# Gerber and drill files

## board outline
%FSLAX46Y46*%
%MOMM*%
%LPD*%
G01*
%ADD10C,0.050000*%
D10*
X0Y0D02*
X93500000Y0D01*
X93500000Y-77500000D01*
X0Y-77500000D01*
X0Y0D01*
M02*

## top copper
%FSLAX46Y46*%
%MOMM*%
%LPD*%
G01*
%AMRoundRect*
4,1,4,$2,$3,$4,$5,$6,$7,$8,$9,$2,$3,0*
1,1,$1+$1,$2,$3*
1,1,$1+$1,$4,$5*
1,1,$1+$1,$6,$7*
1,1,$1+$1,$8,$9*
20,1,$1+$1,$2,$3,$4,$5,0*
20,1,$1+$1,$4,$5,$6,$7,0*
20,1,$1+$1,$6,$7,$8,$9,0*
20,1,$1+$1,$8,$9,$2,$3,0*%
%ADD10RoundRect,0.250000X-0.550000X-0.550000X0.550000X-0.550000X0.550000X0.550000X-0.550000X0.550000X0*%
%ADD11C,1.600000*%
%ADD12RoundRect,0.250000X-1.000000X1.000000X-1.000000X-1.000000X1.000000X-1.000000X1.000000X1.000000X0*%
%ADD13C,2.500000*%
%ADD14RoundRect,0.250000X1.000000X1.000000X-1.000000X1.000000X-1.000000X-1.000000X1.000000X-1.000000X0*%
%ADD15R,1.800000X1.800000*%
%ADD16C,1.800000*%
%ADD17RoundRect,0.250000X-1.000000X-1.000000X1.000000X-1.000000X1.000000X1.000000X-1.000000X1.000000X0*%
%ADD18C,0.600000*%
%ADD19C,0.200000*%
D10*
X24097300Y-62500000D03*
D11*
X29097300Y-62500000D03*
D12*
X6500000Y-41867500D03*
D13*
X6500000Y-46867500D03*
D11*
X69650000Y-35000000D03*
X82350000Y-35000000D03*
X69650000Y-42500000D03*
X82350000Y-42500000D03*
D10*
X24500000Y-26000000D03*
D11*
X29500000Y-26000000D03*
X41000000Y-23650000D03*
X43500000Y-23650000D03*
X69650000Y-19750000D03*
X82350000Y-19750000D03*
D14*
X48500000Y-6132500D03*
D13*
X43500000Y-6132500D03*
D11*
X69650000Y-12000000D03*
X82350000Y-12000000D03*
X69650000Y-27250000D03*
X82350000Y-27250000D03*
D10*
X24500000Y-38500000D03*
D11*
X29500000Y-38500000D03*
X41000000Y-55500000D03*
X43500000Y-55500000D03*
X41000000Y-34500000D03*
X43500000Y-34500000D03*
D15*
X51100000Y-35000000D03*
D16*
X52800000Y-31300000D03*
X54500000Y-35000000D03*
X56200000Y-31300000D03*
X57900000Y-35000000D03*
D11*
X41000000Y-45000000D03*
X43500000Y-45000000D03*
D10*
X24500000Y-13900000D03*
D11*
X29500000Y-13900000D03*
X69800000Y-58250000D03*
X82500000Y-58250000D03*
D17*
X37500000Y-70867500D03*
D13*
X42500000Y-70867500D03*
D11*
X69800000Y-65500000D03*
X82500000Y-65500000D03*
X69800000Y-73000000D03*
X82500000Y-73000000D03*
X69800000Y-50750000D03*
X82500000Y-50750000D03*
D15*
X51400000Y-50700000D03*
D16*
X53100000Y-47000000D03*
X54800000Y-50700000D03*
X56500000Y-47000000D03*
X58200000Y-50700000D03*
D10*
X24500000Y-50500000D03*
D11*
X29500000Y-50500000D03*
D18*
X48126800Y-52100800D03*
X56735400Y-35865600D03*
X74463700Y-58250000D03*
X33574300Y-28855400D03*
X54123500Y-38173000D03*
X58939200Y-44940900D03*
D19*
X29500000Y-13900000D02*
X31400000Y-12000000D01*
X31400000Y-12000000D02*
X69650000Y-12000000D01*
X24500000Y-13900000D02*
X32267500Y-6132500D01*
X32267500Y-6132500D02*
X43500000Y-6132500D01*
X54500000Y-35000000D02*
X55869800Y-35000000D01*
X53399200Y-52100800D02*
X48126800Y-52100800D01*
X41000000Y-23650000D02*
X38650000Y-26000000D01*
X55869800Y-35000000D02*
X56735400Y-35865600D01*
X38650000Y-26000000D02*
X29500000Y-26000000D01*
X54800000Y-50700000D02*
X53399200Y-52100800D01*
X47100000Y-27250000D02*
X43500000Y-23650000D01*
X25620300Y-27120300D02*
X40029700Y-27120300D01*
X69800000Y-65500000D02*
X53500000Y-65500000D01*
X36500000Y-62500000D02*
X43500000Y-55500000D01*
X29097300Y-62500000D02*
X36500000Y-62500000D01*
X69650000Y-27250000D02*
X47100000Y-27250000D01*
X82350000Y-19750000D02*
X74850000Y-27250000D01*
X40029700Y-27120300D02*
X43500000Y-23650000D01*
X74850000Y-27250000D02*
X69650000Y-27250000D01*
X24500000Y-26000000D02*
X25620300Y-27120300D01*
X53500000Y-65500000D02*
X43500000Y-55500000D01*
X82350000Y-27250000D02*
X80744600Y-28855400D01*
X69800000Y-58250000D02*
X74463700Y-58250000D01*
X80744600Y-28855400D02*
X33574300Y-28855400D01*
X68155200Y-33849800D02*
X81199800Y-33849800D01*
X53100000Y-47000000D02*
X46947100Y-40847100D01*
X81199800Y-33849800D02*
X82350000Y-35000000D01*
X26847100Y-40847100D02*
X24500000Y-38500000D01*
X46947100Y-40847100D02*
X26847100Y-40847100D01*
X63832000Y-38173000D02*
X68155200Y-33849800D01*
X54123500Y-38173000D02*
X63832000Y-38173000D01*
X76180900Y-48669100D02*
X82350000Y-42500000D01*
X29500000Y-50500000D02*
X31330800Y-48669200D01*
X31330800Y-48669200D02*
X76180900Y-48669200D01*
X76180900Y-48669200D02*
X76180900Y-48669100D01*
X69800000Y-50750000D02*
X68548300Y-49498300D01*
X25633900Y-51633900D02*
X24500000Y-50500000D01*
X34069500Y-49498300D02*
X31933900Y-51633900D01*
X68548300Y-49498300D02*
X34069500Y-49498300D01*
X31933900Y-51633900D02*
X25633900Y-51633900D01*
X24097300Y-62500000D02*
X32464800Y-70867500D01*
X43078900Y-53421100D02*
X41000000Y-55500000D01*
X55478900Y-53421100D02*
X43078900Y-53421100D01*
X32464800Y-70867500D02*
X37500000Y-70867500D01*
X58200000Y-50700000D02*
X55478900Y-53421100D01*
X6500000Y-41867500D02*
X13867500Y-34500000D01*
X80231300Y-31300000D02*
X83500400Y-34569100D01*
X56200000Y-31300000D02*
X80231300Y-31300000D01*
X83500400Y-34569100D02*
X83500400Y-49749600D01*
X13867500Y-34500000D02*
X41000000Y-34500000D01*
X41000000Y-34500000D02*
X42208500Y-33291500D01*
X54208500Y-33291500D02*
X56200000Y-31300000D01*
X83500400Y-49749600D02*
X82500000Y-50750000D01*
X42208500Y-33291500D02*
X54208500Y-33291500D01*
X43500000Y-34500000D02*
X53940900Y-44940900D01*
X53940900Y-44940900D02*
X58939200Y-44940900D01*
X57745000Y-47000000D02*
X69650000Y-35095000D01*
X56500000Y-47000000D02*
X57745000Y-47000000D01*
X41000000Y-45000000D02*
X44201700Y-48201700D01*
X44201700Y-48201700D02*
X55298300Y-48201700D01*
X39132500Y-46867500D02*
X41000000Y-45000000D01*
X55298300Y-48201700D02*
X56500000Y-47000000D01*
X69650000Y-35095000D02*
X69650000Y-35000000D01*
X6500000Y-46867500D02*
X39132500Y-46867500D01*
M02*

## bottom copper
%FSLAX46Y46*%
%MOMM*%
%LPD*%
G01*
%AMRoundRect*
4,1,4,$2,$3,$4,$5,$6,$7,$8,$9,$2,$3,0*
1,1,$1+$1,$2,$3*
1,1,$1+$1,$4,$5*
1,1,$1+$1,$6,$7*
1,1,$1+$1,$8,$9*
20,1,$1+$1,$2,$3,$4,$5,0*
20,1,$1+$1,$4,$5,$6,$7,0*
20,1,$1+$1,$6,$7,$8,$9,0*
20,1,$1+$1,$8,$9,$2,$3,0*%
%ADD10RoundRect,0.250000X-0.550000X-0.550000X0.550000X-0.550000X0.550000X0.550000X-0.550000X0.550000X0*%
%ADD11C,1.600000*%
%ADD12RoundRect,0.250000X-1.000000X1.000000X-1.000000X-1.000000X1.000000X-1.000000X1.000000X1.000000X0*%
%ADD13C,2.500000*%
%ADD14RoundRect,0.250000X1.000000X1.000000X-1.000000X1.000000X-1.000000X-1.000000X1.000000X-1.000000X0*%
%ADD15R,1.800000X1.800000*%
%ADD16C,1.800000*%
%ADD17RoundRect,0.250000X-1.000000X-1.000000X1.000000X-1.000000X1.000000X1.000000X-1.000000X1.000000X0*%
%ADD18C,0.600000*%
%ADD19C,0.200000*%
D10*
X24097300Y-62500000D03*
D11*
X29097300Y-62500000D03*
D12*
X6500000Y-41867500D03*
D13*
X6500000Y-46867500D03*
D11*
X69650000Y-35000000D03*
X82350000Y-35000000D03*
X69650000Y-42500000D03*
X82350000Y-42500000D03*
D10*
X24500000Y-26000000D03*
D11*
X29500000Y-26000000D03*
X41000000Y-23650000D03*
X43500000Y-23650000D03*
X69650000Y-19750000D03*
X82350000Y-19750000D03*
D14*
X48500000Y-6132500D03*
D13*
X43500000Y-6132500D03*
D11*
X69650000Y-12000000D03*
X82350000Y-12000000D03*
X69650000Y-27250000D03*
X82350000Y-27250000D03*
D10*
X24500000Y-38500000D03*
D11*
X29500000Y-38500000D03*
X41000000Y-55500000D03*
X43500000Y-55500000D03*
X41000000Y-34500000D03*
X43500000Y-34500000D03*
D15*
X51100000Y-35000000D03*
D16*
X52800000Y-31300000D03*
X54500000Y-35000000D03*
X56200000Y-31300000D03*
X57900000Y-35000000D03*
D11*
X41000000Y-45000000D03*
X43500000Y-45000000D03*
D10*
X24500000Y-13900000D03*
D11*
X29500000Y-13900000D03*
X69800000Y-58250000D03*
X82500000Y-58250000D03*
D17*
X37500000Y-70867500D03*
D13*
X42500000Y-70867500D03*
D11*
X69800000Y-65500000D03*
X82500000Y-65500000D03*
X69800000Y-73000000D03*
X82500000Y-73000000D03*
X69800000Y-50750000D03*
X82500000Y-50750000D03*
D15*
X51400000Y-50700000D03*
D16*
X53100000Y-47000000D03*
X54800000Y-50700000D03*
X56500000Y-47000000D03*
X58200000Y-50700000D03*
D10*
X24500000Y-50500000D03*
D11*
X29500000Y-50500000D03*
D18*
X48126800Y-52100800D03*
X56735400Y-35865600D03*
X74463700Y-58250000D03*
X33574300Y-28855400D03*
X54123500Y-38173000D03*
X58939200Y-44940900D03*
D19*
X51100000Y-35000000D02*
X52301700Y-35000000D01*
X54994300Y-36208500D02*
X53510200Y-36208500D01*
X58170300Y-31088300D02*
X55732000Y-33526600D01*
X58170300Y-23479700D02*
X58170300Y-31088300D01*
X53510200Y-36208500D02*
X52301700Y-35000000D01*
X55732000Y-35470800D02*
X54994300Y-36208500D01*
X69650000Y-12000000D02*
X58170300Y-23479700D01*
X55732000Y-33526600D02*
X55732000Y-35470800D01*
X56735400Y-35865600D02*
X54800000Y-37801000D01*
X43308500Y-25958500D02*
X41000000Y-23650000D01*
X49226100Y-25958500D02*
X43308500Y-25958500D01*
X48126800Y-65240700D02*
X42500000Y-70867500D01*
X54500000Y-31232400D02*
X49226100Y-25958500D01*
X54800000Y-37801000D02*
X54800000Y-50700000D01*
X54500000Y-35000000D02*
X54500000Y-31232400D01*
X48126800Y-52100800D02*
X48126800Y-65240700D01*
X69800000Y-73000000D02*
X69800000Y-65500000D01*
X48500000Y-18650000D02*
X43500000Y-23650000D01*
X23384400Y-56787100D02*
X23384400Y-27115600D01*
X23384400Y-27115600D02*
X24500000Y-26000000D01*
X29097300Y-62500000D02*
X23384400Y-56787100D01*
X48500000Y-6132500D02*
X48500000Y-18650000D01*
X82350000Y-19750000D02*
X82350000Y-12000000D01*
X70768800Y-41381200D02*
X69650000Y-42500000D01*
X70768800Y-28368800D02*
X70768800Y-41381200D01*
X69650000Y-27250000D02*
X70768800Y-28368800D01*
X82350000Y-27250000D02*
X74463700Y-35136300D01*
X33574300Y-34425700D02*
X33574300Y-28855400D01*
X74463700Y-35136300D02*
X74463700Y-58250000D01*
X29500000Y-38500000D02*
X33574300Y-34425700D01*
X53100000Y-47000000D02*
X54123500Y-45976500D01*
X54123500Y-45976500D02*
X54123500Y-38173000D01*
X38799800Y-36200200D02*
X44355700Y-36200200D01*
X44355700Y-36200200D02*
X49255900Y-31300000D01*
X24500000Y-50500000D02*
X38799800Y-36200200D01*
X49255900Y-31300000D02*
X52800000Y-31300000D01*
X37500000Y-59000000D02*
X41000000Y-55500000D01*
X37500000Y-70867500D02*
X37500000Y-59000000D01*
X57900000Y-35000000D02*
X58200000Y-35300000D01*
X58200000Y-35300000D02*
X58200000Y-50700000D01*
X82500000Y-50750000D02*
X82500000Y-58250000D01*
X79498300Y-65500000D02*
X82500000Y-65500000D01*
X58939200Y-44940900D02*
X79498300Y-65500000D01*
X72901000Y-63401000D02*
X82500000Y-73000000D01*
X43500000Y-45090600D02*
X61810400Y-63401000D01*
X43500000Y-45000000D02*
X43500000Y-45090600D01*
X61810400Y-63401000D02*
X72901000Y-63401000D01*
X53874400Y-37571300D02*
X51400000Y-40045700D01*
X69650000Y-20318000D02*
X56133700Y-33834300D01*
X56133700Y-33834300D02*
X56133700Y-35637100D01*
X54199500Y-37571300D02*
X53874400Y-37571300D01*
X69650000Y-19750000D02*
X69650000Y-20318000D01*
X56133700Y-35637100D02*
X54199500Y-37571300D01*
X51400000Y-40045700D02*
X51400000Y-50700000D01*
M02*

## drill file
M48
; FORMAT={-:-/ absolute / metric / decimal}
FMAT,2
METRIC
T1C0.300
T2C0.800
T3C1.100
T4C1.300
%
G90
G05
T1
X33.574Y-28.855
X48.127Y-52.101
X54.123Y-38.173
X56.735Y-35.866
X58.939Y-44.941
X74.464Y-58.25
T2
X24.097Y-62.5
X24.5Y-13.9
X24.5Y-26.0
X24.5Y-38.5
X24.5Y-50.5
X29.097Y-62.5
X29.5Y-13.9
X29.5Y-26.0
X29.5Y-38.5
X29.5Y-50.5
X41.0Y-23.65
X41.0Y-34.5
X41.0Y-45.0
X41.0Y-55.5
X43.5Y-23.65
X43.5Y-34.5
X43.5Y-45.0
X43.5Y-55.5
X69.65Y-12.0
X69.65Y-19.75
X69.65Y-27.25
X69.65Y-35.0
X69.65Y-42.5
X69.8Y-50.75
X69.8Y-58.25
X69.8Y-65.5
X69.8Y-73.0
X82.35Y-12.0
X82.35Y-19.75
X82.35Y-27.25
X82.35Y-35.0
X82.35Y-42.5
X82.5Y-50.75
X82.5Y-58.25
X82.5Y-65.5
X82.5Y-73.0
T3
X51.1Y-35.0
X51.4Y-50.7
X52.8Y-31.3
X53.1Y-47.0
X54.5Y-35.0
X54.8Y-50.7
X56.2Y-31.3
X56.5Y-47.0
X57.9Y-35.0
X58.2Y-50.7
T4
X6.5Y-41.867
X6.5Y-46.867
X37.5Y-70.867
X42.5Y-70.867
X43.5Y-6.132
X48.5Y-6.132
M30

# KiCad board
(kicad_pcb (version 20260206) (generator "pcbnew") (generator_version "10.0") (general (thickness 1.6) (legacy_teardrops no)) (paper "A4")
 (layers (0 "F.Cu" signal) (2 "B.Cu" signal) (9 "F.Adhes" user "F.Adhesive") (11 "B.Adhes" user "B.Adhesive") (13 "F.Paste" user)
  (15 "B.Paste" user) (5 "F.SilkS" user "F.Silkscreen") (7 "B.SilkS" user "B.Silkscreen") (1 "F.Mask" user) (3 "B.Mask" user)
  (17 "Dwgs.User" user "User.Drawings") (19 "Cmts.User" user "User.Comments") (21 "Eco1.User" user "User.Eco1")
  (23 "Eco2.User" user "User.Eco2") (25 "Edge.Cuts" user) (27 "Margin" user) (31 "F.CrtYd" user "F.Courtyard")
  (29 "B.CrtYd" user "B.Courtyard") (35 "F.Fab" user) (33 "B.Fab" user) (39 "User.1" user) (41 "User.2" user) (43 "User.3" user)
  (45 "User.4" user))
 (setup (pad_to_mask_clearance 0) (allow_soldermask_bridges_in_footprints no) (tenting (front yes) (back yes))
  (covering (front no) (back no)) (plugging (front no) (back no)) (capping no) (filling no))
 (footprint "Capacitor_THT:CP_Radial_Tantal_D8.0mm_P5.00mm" (layer "F.Cu") (at 24.0973 62.5)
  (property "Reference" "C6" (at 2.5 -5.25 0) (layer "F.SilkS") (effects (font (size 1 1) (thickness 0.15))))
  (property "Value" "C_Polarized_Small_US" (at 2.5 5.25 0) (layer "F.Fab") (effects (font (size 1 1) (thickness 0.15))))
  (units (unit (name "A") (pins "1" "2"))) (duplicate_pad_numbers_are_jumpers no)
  (pad "1" thru_hole roundrect (at 0 0) (size 1.6 1.6) (drill 0.8) (layers "*.Cu" "*.Mask") (remove_unused_layers no)
   (roundrect_rratio 0.15625) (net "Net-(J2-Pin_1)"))
  (pad "2" thru_hole circle (at 5 0) (size 1.6 1.6) (drill 0.8) (layers "*.Cu" "*.Mask") (remove_unused_layers no) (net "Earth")))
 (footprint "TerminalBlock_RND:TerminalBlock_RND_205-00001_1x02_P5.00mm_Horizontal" (layer "F.Cu") (at 6.5 41.8675 -90)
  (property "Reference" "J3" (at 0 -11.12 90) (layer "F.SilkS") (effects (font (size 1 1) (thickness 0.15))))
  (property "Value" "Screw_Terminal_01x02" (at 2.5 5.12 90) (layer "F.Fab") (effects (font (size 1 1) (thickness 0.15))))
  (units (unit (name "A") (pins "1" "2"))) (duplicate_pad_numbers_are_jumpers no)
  (pad "1" thru_hole roundrect (at 0 0 270) (size 2.5 2.5) (drill 1.3) (layers "*.Cu" "*.Mask") (remove_unused_layers no)
   (roundrect_rratio 0.1) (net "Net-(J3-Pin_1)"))
  (pad "2" thru_hole circle (at 5 0 270) (size 2.5 2.5) (drill 1.3) (layers "*.Cu" "*.Mask") (remove_unused_layers no)
   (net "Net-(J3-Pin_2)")))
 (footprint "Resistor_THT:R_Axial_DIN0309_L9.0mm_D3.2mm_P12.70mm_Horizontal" (layer "F.Cu") (at 69.65 35)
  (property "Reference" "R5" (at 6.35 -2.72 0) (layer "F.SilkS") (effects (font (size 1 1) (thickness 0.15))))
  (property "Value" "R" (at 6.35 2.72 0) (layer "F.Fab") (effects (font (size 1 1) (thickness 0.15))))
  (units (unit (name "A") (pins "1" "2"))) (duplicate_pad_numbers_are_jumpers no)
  (pad "1" thru_hole circle (at 0 0) (size 1.6 1.6) (drill 0.8) (layers "*.Cu" "*.Mask") (remove_unused_layers no) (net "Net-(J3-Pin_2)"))
  (pad "2" thru_hole circle (at 12.7 0) (size 1.6 1.6) (drill 0.8) (layers "*.Cu" "*.Mask") (remove_unused_layers no) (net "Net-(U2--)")))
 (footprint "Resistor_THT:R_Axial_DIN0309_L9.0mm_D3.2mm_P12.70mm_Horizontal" (layer "F.Cu") (at 69.65 42.5)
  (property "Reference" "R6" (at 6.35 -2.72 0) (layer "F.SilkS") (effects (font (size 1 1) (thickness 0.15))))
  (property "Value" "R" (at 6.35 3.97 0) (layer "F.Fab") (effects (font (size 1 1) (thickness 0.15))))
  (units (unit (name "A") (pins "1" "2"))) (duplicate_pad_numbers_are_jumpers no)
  (pad "1" thru_hole circle (at 0 0) (size 1.6 1.6) (drill 0.8) (layers "*.Cu" "*.Mask") (remove_unused_layers no) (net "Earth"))
  (pad "2" thru_hole circle (at 12.7 0) (size 1.6 1.6) (drill 0.8) (layers "*.Cu" "*.Mask") (remove_unused_layers no) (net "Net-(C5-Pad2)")))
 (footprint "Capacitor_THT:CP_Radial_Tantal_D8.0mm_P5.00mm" (layer "F.Cu") (at 24.5 26)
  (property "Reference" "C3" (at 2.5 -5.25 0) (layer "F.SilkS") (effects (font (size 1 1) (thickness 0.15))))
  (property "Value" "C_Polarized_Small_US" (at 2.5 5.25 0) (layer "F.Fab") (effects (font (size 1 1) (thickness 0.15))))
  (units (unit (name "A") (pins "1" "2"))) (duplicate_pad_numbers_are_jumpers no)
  (pad "1" thru_hole roundrect (at 0 0) (size 1.6 1.6) (drill 0.8) (layers "*.Cu" "*.Mask") (remove_unused_layers no)
   (roundrect_rratio 0.15625) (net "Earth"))
  (pad "2" thru_hole circle (at 5 0) (size 1.6 1.6) (drill 0.8) (layers "*.Cu" "*.Mask") (remove_unused_layers no) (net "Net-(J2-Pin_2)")))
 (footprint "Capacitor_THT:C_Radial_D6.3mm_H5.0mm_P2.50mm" (layer "F.Cu") (at 41 23.65)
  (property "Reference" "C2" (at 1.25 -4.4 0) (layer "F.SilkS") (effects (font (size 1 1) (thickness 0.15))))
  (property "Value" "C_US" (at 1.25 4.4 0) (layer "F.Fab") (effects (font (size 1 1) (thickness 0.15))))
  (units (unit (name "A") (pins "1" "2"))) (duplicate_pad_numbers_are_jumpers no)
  (pad "1" thru_hole circle (at 0 0) (size 1.6 1.6) (drill 0.8) (layers "*.Cu" "*.Mask") (remove_unused_layers no) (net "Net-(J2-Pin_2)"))
  (pad "2" thru_hole circle (at 2.5 0) (size 1.6 1.6) (drill 0.8) (layers "*.Cu" "*.Mask") (remove_unused_layers no) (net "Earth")))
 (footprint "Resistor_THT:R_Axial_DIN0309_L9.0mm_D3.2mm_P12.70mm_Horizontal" (layer "F.Cu") (at 69.65 19.75)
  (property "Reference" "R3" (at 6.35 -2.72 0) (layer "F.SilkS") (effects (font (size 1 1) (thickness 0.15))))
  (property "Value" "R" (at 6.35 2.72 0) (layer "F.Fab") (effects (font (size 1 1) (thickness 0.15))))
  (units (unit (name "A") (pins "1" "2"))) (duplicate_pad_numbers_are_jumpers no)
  (pad "1" thru_hole circle (at 0 0) (size 1.6 1.6) (drill 0.8) (layers "*.Cu" "*.Mask") (remove_unused_layers no) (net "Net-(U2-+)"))
  (pad "2" thru_hole circle (at 12.7 0) (size 1.6 1.6) (drill 0.8) (layers "*.Cu" "*.Mask") (remove_unused_layers no) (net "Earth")))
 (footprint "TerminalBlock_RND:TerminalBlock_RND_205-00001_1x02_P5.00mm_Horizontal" (layer "F.Cu") (at 48.5 6.1325 180)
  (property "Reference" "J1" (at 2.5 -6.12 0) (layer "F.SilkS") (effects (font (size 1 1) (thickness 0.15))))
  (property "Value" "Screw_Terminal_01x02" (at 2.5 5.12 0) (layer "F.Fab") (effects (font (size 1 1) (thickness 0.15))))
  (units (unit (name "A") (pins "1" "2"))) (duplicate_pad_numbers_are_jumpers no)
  (pad "1" thru_hole roundrect (at 0 0 180) (size 2.5 2.5) (drill 1.3) (layers "*.Cu" "*.Mask") (remove_unused_layers no)
   (roundrect_rratio 0.1) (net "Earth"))
  (pad "2" thru_hole circle (at 5 0 180) (size 2.5 2.5) (drill 1.3) (layers "*.Cu" "*.Mask") (remove_unused_layers no)
   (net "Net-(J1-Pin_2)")))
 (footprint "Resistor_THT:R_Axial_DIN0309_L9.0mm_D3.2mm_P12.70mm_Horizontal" (layer "F.Cu") (at 69.65 12)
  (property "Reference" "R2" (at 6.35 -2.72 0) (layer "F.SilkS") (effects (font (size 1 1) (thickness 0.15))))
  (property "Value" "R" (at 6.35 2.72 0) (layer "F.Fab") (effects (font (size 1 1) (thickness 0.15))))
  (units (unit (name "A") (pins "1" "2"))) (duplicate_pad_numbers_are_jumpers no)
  (pad "1" thru_hole circle (at 0 0) (size 1.6 1.6) (drill 0.8) (layers "*.Cu" "*.Mask") (remove_unused_layers no) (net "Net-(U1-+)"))
  (pad "2" thru_hole circle (at 12.7 0) (size 1.6 1.6) (drill 0.8) (layers "*.Cu" "*.Mask") (remove_unused_layers no) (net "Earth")))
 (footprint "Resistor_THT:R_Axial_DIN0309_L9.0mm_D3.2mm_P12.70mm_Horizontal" (layer "F.Cu") (at 69.65 27.25)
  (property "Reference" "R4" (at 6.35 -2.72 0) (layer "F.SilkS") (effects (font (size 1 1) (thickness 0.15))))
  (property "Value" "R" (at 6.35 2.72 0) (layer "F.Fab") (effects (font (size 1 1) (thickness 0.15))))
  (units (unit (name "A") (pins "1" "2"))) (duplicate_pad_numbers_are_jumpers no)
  (pad "1" thru_hole circle (at 0 0) (size 1.6 1.6) (drill 0.8) (layers "*.Cu" "*.Mask") (remove_unused_layers no) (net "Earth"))
  (pad "2" thru_hole circle (at 12.7 0) (size 1.6 1.6) (drill 0.8) (layers "*.Cu" "*.Mask") (remove_unused_layers no) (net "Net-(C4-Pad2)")))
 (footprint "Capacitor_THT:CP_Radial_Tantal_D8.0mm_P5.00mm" (layer "F.Cu") (at 24.5 38.5)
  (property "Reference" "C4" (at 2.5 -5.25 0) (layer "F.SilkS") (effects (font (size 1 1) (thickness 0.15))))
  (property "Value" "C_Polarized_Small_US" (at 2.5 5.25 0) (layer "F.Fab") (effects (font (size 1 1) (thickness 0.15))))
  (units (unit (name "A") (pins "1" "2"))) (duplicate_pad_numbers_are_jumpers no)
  (pad "1" thru_hole roundrect (at 0 0) (size 1.6 1.6) (drill 0.8) (layers "*.Cu" "*.Mask") (remove_unused_layers no)
   (roundrect_rratio 0.15625) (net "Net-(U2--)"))
  (pad "2" thru_hole circle (at 5 0) (size 1.6 1.6) (drill 0.8) (layers "*.Cu" "*.Mask") (remove_unused_layers no) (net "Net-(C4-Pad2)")))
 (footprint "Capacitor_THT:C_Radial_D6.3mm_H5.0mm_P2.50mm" (layer "F.Cu") (at 41 55.5)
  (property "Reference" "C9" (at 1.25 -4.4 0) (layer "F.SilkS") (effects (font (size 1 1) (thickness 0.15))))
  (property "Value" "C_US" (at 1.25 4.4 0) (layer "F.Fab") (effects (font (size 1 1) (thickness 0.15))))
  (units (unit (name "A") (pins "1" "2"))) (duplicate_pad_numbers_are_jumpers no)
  (pad "1" thru_hole circle (at 0 0) (size 1.6 1.6) (drill 0.8) (layers "*.Cu" "*.Mask") (remove_unused_layers no) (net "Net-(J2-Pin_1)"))
  (pad "2" thru_hole circle (at 2.5 0) (size 1.6 1.6) (drill 0.8) (layers "*.Cu" "*.Mask") (remove_unused_layers no) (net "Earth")))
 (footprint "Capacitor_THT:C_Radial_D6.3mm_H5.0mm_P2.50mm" (layer "F.Cu") (at 41 34.5)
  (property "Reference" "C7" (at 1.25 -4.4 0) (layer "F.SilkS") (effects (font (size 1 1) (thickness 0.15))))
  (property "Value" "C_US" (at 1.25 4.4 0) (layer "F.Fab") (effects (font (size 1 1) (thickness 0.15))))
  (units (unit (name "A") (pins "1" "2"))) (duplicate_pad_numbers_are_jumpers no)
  (pad "1" thru_hole circle (at 0 0) (size 1.6 1.6) (drill 0.8) (layers "*.Cu" "*.Mask") (remove_unused_layers no) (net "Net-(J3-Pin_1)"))
  (pad "2" thru_hole circle (at 2.5 0) (size 1.6 1.6) (drill 0.8) (layers "*.Cu" "*.Mask") (remove_unused_layers no) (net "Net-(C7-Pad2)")))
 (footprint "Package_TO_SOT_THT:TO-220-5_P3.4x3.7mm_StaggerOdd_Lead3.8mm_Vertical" (layer "F.Cu") (at 51.1 35)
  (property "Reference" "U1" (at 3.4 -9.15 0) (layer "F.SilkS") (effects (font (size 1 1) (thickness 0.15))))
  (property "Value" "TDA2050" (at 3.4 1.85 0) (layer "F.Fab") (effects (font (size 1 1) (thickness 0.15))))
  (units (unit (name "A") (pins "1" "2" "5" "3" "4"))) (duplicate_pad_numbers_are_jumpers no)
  (pad "1" thru_hole rect (at 0 0) (size 1.8 1.8) (drill 1.1) (layers "*.Cu" "*.Mask") (remove_unused_layers no) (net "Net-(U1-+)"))
  (pad "2" thru_hole circle (at 1.7 -3.7) (size 1.8 1.8) (drill 1.1) (layers "*.Cu" "*.Mask") (remove_unused_layers no) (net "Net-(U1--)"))
  (pad "3" thru_hole circle (at 3.4 0) (size 1.8 1.8) (drill 1.1) (layers "*.Cu" "*.Mask") (remove_unused_layers no) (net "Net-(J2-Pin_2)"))
  (pad "4" thru_hole circle (at 5.1 -3.7) (size 1.8 1.8) (drill 1.1) (layers "*.Cu" "*.Mask") (remove_unused_layers no)
   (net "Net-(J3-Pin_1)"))
  (pad "5" thru_hole circle (at 6.8 0) (size 1.8 1.8) (drill 1.1) (layers "*.Cu" "*.Mask") (remove_unused_layers no) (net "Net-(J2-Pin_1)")))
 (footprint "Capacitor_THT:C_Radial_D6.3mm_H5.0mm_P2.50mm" (layer "F.Cu") (at 41 45)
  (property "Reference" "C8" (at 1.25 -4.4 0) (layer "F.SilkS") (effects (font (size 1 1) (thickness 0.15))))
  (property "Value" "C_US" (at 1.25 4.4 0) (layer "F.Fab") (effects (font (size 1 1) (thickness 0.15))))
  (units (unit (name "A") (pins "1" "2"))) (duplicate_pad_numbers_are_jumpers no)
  (pad "1" thru_hole circle (at 0 0) (size 1.6 1.6) (drill 0.8) (layers "*.Cu" "*.Mask") (remove_unused_layers no) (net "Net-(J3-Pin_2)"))
  (pad "2" thru_hole circle (at 2.5 0) (size 1.6 1.6) (drill 0.8) (layers "*.Cu" "*.Mask") (remove_unused_layers no) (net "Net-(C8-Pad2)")))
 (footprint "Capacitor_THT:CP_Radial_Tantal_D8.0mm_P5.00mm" (layer "F.Cu") (at 24.5 13.9)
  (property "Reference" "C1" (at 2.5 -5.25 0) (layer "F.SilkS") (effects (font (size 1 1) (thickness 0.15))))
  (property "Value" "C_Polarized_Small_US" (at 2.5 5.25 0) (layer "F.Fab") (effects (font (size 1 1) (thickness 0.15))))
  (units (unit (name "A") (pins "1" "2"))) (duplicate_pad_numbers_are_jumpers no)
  (pad "1" thru_hole roundrect (at 0 0) (size 1.6 1.6) (drill 0.8) (layers "*.Cu" "*.Mask") (remove_unused_layers no)
   (roundrect_rratio 0.15625) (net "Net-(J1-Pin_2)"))
  (pad "2" thru_hole circle (at 5 0) (size 1.6 1.6) (drill 0.8) (layers "*.Cu" "*.Mask") (remove_unused_layers no) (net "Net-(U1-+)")))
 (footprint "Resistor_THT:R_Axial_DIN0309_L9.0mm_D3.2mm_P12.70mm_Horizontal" (layer "F.Cu") (at 69.8 58.25)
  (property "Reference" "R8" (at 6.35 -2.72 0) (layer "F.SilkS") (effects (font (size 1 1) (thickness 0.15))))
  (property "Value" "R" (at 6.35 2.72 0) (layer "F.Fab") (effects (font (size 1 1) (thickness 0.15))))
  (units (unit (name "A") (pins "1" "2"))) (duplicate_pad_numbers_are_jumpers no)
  (pad "1" thru_hole circle (at 0 0) (size 1.6 1.6) (drill 0.8) (layers "*.Cu" "*.Mask") (remove_unused_layers no) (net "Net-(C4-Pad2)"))
  (pad "2" thru_hole circle (at 12.7 0) (size 1.6 1.6) (drill 0.8) (layers "*.Cu" "*.Mask") (remove_unused_layers no) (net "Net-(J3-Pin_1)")))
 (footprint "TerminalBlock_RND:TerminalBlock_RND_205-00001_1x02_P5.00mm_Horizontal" (layer "F.Cu") (at 37.5 70.8675)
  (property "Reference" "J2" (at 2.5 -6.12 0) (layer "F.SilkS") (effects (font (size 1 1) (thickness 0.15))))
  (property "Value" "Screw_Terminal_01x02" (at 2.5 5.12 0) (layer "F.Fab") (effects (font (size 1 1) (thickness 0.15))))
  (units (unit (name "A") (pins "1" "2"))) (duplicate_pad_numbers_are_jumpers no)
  (pad "1" thru_hole roundrect (at 0 0) (size 2.5 2.5) (drill 1.3) (layers "*.Cu" "*.Mask") (remove_unused_layers no) (roundrect_rratio 0.1)
   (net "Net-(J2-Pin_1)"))
  (pad "2" thru_hole circle (at 5 0) (size 2.5 2.5) (drill 1.3) (layers "*.Cu" "*.Mask") (remove_unused_layers no) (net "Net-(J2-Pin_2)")))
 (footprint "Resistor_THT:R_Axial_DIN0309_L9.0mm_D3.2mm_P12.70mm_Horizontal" (layer "F.Cu") (at 69.8 65.5)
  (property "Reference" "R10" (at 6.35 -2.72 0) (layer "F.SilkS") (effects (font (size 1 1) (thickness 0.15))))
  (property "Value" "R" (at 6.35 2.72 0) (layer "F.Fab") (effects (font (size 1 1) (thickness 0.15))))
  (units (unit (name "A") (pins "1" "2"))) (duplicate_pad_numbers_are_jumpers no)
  (pad "1" thru_hole circle (at 0 0) (size 1.6 1.6) (drill 0.8) (layers "*.Cu" "*.Mask") (remove_unused_layers no) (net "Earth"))
  (pad "2" thru_hole circle (at 12.7 0) (size 1.6 1.6) (drill 0.8) (layers "*.Cu" "*.Mask") (remove_unused_layers no) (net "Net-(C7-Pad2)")))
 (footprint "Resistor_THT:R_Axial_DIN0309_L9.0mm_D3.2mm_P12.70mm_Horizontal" (layer "F.Cu") (at 69.8 73)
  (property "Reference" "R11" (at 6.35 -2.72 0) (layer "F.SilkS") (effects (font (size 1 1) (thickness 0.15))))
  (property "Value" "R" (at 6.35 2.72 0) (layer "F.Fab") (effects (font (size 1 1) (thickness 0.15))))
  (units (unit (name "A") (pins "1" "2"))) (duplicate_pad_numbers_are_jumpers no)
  (pad "1" thru_hole circle (at 0 0) (size 1.6 1.6) (drill 0.8) (layers "*.Cu" "*.Mask") (remove_unused_layers no) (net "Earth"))
  (pad "2" thru_hole circle (at 12.7 0) (size 1.6 1.6) (drill 0.8) (layers "*.Cu" "*.Mask") (remove_unused_layers no) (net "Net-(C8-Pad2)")))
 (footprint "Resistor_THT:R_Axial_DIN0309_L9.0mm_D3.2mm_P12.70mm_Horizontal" (layer "F.Cu") (at 69.8 50.75)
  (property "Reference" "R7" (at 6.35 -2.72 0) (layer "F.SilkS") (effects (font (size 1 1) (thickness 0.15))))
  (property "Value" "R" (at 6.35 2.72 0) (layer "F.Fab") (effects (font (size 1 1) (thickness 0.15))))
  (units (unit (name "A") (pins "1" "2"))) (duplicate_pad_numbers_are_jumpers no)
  (pad "1" thru_hole circle (at 0 0) (size 1.6 1.6) (drill 0.8) (layers "*.Cu" "*.Mask") (remove_unused_layers no) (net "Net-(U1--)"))
  (pad "2" thru_hole circle (at 12.7 0) (size 1.6 1.6) (drill 0.8) (layers "*.Cu" "*.Mask") (remove_unused_layers no) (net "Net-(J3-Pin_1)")))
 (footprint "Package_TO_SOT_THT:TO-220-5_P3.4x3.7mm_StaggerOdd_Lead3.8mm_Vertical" (layer "F.Cu") (at 51.4 50.7)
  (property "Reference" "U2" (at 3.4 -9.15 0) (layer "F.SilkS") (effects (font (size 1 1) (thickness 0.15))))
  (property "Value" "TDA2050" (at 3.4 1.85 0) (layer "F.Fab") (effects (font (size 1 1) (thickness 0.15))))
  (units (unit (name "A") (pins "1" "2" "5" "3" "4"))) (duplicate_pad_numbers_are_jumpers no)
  (pad "1" thru_hole rect (at 0 0) (size 1.8 1.8) (drill 1.1) (layers "*.Cu" "*.Mask") (remove_unused_layers no) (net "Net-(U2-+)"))
  (pad "2" thru_hole circle (at 1.7 -3.7) (size 1.8 1.8) (drill 1.1) (layers "*.Cu" "*.Mask") (remove_unused_layers no) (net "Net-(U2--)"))
  (pad "3" thru_hole circle (at 3.4 0) (size 1.8 1.8) (drill 1.1) (layers "*.Cu" "*.Mask") (remove_unused_layers no) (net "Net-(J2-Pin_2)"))
  (pad "4" thru_hole circle (at 5.1 -3.7) (size 1.8 1.8) (drill 1.1) (layers "*.Cu" "*.Mask") (remove_unused_layers no)
   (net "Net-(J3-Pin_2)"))
  (pad "5" thru_hole circle (at 6.8 0) (size 1.8 1.8) (drill 1.1) (layers "*.Cu" "*.Mask") (remove_unused_layers no) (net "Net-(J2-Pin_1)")))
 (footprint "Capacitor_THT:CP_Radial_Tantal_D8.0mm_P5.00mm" (layer "F.Cu") (at 24.5 50.5)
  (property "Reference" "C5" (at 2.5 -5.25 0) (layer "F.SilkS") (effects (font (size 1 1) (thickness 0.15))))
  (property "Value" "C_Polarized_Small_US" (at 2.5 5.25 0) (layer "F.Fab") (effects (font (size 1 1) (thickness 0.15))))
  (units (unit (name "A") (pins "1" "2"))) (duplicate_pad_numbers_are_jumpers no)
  (pad "1" thru_hole roundrect (at 0 0) (size 1.6 1.6) (drill 0.8) (layers "*.Cu" "*.Mask") (remove_unused_layers no)
   (roundrect_rratio 0.15625) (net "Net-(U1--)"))
  (pad "2" thru_hole circle (at 5 0) (size 1.6 1.6) (drill 0.8) (layers "*.Cu" "*.Mask") (remove_unused_layers no) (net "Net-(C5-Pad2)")))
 (gr_rect (start 0 0) (end 93.5 77.5) (stroke (width 0.05) (type default)) (fill no) (layer "Edge.Cuts"))
 (segment (start 29.5 13.9) (end 31.4 12) (width 0.2) (layer "F.Cu") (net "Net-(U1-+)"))
 (segment (start 31.4 12) (end 69.65 12) (width 0.2) (layer "F.Cu") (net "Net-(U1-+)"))
 (segment (start 51.1 35) (end 52.3017 35) (width 0.2) (layer "B.Cu") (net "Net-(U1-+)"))
 (segment (start 54.9943 36.2085) (end 53.5102 36.2085) (width 0.2) (layer "B.Cu") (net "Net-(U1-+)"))
 (segment (start 58.1703 31.0883) (end 55.732 33.5266) (width 0.2) (layer "B.Cu") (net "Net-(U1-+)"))
 (segment (start 58.1703 23.4797) (end 58.1703 31.0883) (width 0.2) (layer "B.Cu") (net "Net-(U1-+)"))
 (segment (start 53.5102 36.2085) (end 52.3017 35) (width 0.2) (layer "B.Cu") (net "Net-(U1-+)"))
 (segment (start 55.732 35.4708) (end 54.9943 36.2085) (width 0.2) (layer "B.Cu") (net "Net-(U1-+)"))
 (segment (start 69.65 12) (end 58.1703 23.4797) (width 0.2) (layer "B.Cu") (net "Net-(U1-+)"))
 (segment (start 55.732 33.5266) (end 55.732 35.4708) (width 0.2) (layer "B.Cu") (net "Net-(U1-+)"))
 (segment (start 24.5 13.9) (end 32.2675 6.1325) (width 0.2) (layer "F.Cu") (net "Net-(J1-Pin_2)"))
 (segment (start 32.2675 6.1325) (end 43.5 6.1325) (width 0.2) (layer "F.Cu") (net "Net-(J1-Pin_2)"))
 (segment (start 54.5 35) (end 55.8698 35) (width 0.2) (layer "F.Cu") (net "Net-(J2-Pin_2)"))
 (segment (start 53.3992 52.1008) (end 48.1268 52.1008) (width 0.2) (layer "F.Cu") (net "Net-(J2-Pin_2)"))
 (segment (start 41 23.65) (end 38.65 26) (width 0.2) (layer "F.Cu") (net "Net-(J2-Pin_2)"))
 (segment (start 55.8698 35) (end 56.7354 35.8656) (width 0.2) (layer "F.Cu") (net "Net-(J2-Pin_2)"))
 (segment (start 38.65 26) (end 29.5 26) (width 0.2) (layer "F.Cu") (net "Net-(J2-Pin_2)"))
 (segment (start 54.8 50.7) (end 53.3992 52.1008) (width 0.2) (layer "F.Cu") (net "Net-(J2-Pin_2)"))
 (via (at 48.1268 52.1008) (size 0.6) (drill 0.3) (layers "F.Cu" "B.Cu") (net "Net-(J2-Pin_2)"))
 (via (at 56.7354 35.8656) (size 0.6) (drill 0.3) (layers "F.Cu" "B.Cu") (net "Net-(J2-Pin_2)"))
 (segment (start 56.7354 35.8656) (end 54.8 37.801) (width 0.2) (layer "B.Cu") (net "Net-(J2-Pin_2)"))
 (segment (start 43.3085 25.9585) (end 41 23.65) (width 0.2) (layer "B.Cu") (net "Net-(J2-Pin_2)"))
 (segment (start 49.2261 25.9585) (end 43.3085 25.9585) (width 0.2) (layer "B.Cu") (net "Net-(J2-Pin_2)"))
 (segment (start 48.1268 65.2407) (end 42.5 70.8675) (width 0.2) (layer "B.Cu") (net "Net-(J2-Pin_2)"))
 (segment (start 54.5 31.2324) (end 49.2261 25.9585) (width 0.2) (layer "B.Cu") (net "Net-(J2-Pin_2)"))
 (segment (start 54.8 37.801) (end 54.8 50.7) (width 0.2) (layer "B.Cu") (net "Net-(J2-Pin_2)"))
 (segment (start 54.5 35) (end 54.5 31.2324) (width 0.2) (layer "B.Cu") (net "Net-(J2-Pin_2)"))
 (segment (start 48.1268 52.1008) (end 48.1268 65.2407) (width 0.2) (layer "B.Cu") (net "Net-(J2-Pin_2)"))
 (segment (start 47.1 27.25) (end 43.5 23.65) (width 0.2) (layer "F.Cu") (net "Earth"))
 (segment (start 25.6203 27.1203) (end 40.0297 27.1203) (width 0.2) (layer "F.Cu") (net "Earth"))
 (segment (start 69.8 65.5) (end 53.5 65.5) (width 0.2) (layer "F.Cu") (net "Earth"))
 (segment (start 36.5 62.5) (end 43.5 55.5) (width 0.2) (layer "F.Cu") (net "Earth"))
 (segment (start 29.0973 62.5) (end 36.5 62.5) (width 0.2) (layer "F.Cu") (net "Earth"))
 (segment (start 69.65 27.25) (end 47.1 27.25) (width 0.2) (layer "F.Cu") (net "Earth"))
 (segment (start 82.35 19.75) (end 74.85 27.25) (width 0.2) (layer "F.Cu") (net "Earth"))
 (segment (start 40.0297 27.1203) (end 43.5 23.65) (width 0.2) (layer "F.Cu") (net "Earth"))
 (segment (start 74.85 27.25) (end 69.65 27.25) (width 0.2) (layer "F.Cu") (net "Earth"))
 (segment (start 24.5 26) (end 25.6203 27.1203) (width 0.2) (layer "F.Cu") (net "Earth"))
 (segment (start 53.5 65.5) (end 43.5 55.5) (width 0.2) (layer "F.Cu") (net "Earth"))
 (segment (start 69.8 73) (end 69.8 65.5) (width 0.2) (layer "B.Cu") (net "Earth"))
 (segment (start 48.5 18.65) (end 43.5 23.65) (width 0.2) (layer "B.Cu") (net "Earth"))
 (segment (start 23.3844 56.7871) (end 23.3844 27.1156) (width 0.2) (layer "B.Cu") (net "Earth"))
 (segment (start 23.3844 27.1156) (end 24.5 26) (width 0.2) (layer "B.Cu") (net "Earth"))
 (segment (start 29.0973 62.5) (end 23.3844 56.7871) (width 0.2) (layer "B.Cu") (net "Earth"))
 (segment (start 48.5 6.1325) (end 48.5 18.65) (width 0.2) (layer "B.Cu") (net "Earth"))
 (segment (start 82.35 19.75) (end 82.35 12) (width 0.2) (layer "B.Cu") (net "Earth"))
 (segment (start 70.7688 41.3812) (end 69.65 42.5) (width 0.2) (layer "B.Cu") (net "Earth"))
 (segment (start 70.7688 28.3688) (end 70.7688 41.3812) (width 0.2) (layer "B.Cu") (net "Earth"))
 (segment (start 69.65 27.25) (end 70.7688 28.3688) (width 0.2) (layer "B.Cu") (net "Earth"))
 (segment (start 82.35 27.25) (end 80.7446 28.8554) (width 0.2) (layer "F.Cu") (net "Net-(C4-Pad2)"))
 (segment (start 69.8 58.25) (end 74.4637 58.25) (width 0.2) (layer "F.Cu") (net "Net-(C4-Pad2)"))
 (segment (start 80.7446 28.8554) (end 33.5743 28.8554) (width 0.2) (layer "F.Cu") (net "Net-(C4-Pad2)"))
 (via (at 74.4637 58.25) (size 0.6) (drill 0.3) (layers "F.Cu" "B.Cu") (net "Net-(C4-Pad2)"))
 (via (at 33.5743 28.8554) (size 0.6) (drill 0.3) (layers "F.Cu" "B.Cu") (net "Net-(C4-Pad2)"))
 (segment (start 82.35 27.25) (end 74.4637 35.1363) (width 0.2) (layer "B.Cu") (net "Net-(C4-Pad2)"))
 (segment (start 33.5743 34.4257) (end 33.5743 28.8554) (width 0.2) (layer "B.Cu") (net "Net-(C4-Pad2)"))
 (segment (start 74.4637 35.1363) (end 74.4637 58.25) (width 0.2) (layer "B.Cu") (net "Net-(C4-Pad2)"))
 (segment (start 29.5 38.5) (end 33.5743 34.4257) (width 0.2) (layer "B.Cu") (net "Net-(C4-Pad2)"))
 (segment (start 68.1552 33.8498) (end 81.1998 33.8498) (width 0.2) (layer "F.Cu") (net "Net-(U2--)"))
 (segment (start 53.1 47) (end 46.9471 40.8471) (width 0.2) (layer "F.Cu") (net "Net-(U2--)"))
 (segment (start 81.1998 33.8498) (end 82.35 35) (width 0.2) (layer "F.Cu") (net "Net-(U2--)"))
 (segment (start 26.8471 40.8471) (end 24.5 38.5) (width 0.2) (layer "F.Cu") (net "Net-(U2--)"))
 (segment (start 46.9471 40.8471) (end 26.8471 40.8471) (width 0.2) (layer "F.Cu") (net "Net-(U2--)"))
 (segment (start 63.832 38.173) (end 68.1552 33.8498) (width 0.2) (layer "F.Cu") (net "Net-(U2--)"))
 (segment (start 54.1235 38.173) (end 63.832 38.173) (width 0.2) (layer "F.Cu") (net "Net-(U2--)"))
 (via (at 54.1235 38.173) (size 0.6) (drill 0.3) (layers "F.Cu" "B.Cu") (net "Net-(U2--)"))
 (segment (start 53.1 47) (end 54.1235 45.9765) (width 0.2) (layer "B.Cu") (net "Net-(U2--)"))
 (segment (start 54.1235 45.9765) (end 54.1235 38.173) (width 0.2) (layer "B.Cu") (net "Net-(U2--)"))
 (segment (start 76.1809 48.6691) (end 82.35 42.5) (width 0.2) (layer "F.Cu") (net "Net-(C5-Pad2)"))
 (segment (start 29.5 50.5) (end 31.3308 48.6692) (width 0.2) (layer "F.Cu") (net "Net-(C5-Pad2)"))
 (segment (start 31.3308 48.6692) (end 76.1809 48.6692) (width 0.2) (layer "F.Cu") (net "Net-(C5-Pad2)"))
 (segment (start 76.1809 48.6692) (end 76.1809 48.6691) (width 0.2) (layer "F.Cu") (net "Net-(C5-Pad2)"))
 (segment (start 69.8 50.75) (end 68.5483 49.4983) (width 0.2) (layer "F.Cu") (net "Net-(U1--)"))
 (segment (start 25.6339 51.6339) (end 24.5 50.5) (width 0.2) (layer "F.Cu") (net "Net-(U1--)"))
 (segment (start 34.0695 49.4983) (end 31.9339 51.6339) (width 0.2) (layer "F.Cu") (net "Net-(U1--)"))
 (segment (start 68.5483 49.4983) (end 34.0695 49.4983) (width 0.2) (layer "F.Cu") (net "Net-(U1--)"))
 (segment (start 31.9339 51.6339) (end 25.6339 51.6339) (width 0.2) (layer "F.Cu") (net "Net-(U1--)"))
 (segment (start 38.7998 36.2002) (end 44.3557 36.2002) (width 0.2) (layer "B.Cu") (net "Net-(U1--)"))
 (segment (start 44.3557 36.2002) (end 49.2559 31.3) (width 0.2) (layer "B.Cu") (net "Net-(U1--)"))
 (segment (start 24.5 50.5) (end 38.7998 36.2002) (width 0.2) (layer "B.Cu") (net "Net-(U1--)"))
 (segment (start 49.2559 31.3) (end 52.8 31.3) (width 0.2) (layer "B.Cu") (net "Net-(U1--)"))
 (segment (start 24.0973 62.5) (end 32.4648 70.8675) (width 0.2) (layer "F.Cu") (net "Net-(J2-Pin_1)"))
 (segment (start 43.0789 53.4211) (end 41 55.5) (width 0.2) (layer "F.Cu") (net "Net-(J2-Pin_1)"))
 (segment (start 55.4789 53.4211) (end 43.0789 53.4211) (width 0.2) (layer "F.Cu") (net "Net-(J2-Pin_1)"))
 (segment (start 32.4648 70.8675) (end 37.5 70.8675) (width 0.2) (layer "F.Cu") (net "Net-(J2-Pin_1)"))
 (segment (start 58.2 50.7) (end 55.4789 53.4211) (width 0.2) (layer "F.Cu") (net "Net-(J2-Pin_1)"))
 (segment (start 37.5 59) (end 41 55.5) (width 0.2) (layer "B.Cu") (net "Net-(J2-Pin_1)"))
 (segment (start 37.5 70.8675) (end 37.5 59) (width 0.2) (layer "B.Cu") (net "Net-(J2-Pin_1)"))
 (segment (start 57.9 35) (end 58.2 35.3) (width 0.2) (layer "B.Cu") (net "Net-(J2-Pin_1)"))
 (segment (start 58.2 35.3) (end 58.2 50.7) (width 0.2) (layer "B.Cu") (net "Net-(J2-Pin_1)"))
 (segment (start 6.5 41.8675) (end 13.8675 34.5) (width 0.2) (layer "F.Cu") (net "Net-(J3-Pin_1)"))
 (segment (start 80.2313 31.3) (end 83.5004 34.5691) (width 0.2) (layer "F.Cu") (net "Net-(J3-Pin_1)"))
 (segment (start 56.2 31.3) (end 80.2313 31.3) (width 0.2) (layer "F.Cu") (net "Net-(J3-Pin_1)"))
 (segment (start 83.5004 34.5691) (end 83.5004 49.7496) (width 0.2) (layer "F.Cu") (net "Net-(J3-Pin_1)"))
 (segment (start 13.8675 34.5) (end 41 34.5) (width 0.2) (layer "F.Cu") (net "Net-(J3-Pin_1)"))
 (segment (start 41 34.5) (end 42.2085 33.2915) (width 0.2) (layer "F.Cu") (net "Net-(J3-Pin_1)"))
 (segment (start 54.2085 33.2915) (end 56.2 31.3) (width 0.2) (layer "F.Cu") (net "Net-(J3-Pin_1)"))
 (segment (start 83.5004 49.7496) (end 82.5 50.75) (width 0.2) (layer "F.Cu") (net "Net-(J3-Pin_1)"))
 (segment (start 42.2085 33.2915) (end 54.2085 33.2915) (width 0.2) (layer "F.Cu") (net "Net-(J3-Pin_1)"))
 (segment (start 82.5 50.75) (end 82.5 58.25) (width 0.2) (layer "B.Cu") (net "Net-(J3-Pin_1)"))
 (segment (start 43.5 34.5) (end 53.9409 44.9409) (width 0.2) (layer "F.Cu") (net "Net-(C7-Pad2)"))
 (segment (start 53.9409 44.9409) (end 58.9392 44.9409) (width 0.2) (layer "F.Cu") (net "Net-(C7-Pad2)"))
 (via (at 58.9392 44.9409) (size 0.6) (drill 0.3) (layers "F.Cu" "B.Cu") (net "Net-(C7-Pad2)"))
 (segment (start 79.4983 65.5) (end 82.5 65.5) (width 0.2) (layer "B.Cu") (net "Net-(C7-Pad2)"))
 (segment (start 58.9392 44.9409) (end 79.4983 65.5) (width 0.2) (layer "B.Cu") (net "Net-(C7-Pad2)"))
 (segment (start 57.745 47) (end 69.65 35.095) (width 0.2) (layer "F.Cu") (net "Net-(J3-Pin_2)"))
 (segment (start 56.5 47) (end 57.745 47) (width 0.2) (layer "F.Cu") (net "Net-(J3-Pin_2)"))
 (segment (start 41 45) (end 44.2017 48.2017) (width 0.2) (layer "F.Cu") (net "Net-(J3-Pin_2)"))
 (segment (start 44.2017 48.2017) (end 55.2983 48.2017) (width 0.2) (layer "F.Cu") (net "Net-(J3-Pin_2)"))
 (segment (start 39.1325 46.8675) (end 41 45) (width 0.2) (layer "F.Cu") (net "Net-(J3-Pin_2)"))
 (segment (start 55.2983 48.2017) (end 56.5 47) (width 0.2) (layer "F.Cu") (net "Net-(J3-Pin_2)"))
 (segment (start 69.65 35.095) (end 69.65 35) (width 0.2) (layer "F.Cu") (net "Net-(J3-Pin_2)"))
 (segment (start 6.5 46.8675) (end 39.1325 46.8675) (width 0.2) (layer "F.Cu") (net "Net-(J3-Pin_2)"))
 (segment (start 72.901 63.401) (end 82.5 73) (width 0.2) (layer "B.Cu") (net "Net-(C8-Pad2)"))
 (segment (start 43.5 45.0906) (end 61.8104 63.401) (width 0.2) (layer "B.Cu") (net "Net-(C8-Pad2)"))
 (segment (start 43.5 45) (end 43.5 45.0906) (width 0.2) (layer "B.Cu") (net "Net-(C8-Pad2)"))
 (segment (start 61.8104 63.401) (end 72.901 63.401) (width 0.2) (layer "B.Cu") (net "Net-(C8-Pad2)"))
 (segment (start 53.8744 37.5713) (end 51.4 40.0457) (width 0.2) (layer "B.Cu") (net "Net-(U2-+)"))
 (segment (start 69.65 20.318) (end 56.1337 33.8343) (width 0.2) (layer "B.Cu") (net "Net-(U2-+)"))
 (segment (start 56.1337 33.8343) (end 56.1337 35.6371) (width 0.2) (layer "B.Cu") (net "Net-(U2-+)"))
 (segment (start 54.1995 37.5713) (end 53.8744 37.5713) (width 0.2) (layer "B.Cu") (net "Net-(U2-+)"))
 (segment (start 69.65 19.75) (end 69.65 20.318) (width 0.2) (layer "B.Cu") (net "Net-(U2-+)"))
 (segment (start 56.1337 35.6371) (end 54.1995 37.5713) (width 0.2) (layer "B.Cu") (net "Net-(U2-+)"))
 (segment (start 51.4 40.0457) (end 51.4 50.7) (width 0.2) (layer "B.Cu") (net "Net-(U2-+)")))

